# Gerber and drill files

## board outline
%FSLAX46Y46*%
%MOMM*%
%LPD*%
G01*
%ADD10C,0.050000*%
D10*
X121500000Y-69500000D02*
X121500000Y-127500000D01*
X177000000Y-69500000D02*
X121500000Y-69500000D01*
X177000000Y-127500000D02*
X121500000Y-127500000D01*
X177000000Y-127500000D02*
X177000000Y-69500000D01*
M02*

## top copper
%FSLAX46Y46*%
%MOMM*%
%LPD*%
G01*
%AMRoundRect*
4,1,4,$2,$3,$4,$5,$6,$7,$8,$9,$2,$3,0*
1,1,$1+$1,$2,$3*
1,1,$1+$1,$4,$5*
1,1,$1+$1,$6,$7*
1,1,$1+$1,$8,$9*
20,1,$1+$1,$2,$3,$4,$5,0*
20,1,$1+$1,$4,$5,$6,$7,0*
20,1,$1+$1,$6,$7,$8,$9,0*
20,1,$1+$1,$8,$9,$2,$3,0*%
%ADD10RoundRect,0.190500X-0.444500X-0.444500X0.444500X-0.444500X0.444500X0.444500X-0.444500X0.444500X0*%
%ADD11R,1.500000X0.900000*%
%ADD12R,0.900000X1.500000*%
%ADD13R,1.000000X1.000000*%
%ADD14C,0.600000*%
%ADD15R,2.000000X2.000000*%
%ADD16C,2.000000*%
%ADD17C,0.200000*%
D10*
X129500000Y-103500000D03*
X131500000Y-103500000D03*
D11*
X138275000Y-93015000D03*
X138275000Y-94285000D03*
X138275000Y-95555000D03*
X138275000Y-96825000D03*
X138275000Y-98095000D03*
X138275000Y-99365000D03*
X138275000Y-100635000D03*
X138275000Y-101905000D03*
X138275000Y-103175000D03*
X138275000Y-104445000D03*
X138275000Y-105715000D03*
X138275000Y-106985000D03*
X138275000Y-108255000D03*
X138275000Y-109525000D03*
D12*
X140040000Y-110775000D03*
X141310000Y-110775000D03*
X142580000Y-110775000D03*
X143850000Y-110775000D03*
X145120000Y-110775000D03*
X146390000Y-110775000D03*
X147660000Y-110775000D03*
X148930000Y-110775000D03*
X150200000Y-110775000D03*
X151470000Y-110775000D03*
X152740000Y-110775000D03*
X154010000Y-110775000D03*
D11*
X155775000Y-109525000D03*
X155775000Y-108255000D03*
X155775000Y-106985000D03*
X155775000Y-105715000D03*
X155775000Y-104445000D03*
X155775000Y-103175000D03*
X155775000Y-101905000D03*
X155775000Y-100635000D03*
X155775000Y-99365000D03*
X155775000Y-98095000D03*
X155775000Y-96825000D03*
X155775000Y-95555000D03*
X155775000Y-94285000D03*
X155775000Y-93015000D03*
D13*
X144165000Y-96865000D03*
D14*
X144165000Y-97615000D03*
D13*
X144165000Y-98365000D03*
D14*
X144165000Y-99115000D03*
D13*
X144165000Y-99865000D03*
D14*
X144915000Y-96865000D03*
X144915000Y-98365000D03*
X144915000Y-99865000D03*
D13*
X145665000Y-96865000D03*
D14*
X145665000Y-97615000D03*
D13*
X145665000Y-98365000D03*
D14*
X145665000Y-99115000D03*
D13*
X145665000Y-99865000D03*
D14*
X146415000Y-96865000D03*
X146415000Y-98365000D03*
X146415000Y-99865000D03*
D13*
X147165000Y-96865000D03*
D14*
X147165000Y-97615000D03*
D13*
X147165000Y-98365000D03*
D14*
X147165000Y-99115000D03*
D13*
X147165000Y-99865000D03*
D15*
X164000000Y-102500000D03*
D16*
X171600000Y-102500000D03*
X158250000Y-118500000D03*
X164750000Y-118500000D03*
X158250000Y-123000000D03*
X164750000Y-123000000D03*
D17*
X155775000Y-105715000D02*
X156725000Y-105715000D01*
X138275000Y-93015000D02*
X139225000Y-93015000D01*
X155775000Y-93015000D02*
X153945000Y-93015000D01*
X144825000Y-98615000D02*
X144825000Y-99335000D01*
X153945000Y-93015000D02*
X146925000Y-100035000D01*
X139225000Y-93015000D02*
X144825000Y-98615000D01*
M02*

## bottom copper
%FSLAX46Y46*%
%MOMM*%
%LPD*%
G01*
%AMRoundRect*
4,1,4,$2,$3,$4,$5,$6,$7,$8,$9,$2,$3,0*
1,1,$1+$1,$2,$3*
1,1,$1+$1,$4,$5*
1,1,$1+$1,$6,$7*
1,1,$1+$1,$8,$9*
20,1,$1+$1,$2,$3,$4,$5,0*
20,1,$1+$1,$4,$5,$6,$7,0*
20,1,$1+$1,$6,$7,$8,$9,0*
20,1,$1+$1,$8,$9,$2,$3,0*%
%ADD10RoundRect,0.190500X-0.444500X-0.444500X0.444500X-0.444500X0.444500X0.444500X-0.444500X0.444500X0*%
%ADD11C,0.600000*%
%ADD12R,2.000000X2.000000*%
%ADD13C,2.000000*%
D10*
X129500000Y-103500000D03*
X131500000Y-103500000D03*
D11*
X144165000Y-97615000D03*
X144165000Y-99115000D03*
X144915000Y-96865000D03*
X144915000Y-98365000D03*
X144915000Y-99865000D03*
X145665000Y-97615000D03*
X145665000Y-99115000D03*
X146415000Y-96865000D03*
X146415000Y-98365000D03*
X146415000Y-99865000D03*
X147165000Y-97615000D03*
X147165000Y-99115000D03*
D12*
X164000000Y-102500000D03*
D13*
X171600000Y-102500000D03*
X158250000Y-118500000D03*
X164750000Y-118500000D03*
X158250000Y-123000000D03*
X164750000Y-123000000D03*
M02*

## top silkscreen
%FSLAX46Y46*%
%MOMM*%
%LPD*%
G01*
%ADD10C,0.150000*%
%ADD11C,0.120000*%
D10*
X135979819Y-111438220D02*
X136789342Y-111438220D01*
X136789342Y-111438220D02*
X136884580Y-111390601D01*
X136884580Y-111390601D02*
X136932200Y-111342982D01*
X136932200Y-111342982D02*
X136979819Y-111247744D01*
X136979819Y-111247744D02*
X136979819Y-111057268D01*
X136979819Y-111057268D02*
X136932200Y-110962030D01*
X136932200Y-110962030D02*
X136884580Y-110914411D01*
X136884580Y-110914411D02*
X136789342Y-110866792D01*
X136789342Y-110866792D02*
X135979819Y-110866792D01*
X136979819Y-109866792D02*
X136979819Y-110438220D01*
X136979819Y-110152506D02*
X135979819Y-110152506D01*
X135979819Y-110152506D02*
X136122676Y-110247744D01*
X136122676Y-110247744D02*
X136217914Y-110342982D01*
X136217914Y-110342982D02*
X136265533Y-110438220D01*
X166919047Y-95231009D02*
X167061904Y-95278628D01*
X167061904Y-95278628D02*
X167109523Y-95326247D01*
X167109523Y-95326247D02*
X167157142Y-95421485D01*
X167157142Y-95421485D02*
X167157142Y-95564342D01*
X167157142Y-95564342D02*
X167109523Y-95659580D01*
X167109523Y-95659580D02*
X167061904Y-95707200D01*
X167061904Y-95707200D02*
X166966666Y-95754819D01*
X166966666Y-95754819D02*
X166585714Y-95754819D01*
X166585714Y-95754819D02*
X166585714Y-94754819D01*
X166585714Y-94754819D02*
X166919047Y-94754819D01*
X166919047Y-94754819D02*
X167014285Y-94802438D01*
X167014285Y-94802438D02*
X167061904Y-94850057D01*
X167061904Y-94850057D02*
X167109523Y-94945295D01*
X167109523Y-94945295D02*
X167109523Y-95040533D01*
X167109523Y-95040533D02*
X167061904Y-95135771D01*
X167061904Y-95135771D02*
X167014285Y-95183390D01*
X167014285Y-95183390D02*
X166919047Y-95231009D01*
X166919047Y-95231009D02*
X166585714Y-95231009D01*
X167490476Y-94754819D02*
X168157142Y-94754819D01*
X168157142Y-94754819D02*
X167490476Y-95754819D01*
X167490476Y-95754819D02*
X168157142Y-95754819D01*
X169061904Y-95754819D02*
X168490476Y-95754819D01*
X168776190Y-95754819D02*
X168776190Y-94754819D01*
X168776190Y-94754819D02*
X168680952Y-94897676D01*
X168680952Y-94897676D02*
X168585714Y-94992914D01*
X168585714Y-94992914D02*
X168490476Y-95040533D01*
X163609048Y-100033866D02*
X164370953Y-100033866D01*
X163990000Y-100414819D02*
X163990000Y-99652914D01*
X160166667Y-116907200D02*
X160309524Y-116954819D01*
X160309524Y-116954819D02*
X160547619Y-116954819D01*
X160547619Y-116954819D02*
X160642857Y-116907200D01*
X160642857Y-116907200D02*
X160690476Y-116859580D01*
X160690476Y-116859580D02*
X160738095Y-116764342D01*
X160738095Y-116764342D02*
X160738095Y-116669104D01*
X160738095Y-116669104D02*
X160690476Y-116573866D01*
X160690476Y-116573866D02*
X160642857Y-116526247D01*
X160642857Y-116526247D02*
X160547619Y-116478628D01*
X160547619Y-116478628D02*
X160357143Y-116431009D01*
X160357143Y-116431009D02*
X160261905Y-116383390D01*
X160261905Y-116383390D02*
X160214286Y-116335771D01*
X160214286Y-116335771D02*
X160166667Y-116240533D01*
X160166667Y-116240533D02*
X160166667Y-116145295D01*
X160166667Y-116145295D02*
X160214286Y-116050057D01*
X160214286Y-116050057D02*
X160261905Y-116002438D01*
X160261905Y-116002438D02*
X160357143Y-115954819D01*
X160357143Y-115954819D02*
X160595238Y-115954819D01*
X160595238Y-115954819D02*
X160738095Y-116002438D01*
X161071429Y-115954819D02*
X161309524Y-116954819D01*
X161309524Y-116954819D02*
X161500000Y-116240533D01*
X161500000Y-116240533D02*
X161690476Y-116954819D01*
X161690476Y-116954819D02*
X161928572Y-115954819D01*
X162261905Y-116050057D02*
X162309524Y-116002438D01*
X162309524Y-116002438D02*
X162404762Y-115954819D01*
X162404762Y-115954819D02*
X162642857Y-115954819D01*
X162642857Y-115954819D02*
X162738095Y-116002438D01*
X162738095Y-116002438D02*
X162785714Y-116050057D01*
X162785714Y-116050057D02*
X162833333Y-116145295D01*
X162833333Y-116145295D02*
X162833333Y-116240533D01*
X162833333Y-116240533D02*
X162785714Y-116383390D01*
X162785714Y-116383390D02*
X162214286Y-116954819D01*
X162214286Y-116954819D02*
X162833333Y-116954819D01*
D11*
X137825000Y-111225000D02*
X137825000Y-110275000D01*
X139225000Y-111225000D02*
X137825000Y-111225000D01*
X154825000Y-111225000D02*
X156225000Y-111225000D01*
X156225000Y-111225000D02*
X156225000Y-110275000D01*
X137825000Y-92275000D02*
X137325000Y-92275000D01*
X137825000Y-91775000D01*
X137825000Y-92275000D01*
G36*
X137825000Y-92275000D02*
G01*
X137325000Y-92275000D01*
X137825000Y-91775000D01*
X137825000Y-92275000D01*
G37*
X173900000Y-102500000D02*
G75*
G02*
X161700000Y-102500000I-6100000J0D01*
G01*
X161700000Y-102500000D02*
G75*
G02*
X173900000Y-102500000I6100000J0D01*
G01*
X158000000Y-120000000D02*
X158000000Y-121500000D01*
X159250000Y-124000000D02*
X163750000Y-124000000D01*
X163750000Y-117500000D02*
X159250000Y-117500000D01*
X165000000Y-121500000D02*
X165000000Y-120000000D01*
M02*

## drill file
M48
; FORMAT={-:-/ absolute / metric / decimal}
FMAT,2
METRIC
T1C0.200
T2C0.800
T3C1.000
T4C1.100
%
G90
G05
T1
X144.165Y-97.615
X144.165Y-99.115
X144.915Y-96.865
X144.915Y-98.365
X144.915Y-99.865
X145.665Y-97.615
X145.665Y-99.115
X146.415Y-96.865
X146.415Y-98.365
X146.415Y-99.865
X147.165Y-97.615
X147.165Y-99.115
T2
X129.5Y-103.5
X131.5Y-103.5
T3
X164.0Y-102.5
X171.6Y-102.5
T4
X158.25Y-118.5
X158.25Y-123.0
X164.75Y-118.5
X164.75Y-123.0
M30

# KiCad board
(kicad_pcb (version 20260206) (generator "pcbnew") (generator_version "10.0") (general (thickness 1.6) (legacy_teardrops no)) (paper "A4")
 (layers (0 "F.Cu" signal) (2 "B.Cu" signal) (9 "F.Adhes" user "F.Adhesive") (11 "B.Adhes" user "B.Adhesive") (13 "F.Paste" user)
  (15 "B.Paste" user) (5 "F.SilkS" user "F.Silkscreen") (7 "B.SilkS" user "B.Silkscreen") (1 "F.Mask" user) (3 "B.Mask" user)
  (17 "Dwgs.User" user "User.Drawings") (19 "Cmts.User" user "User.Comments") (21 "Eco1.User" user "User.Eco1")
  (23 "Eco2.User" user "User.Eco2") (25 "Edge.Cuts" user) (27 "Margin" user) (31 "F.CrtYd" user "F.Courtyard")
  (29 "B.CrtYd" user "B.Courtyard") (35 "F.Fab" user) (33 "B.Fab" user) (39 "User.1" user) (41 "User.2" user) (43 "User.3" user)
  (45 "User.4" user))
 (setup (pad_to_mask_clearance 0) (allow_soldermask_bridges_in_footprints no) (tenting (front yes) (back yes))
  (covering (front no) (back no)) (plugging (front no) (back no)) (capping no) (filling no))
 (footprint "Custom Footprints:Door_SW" (layer "F.Cu") (at 130.5 107.5)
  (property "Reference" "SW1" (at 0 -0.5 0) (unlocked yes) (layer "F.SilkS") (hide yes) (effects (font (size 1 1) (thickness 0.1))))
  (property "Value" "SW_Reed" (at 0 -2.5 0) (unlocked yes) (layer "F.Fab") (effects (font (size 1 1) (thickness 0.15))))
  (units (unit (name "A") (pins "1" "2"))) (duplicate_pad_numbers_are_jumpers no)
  (pad "1" thru_hole roundrect (at -1 -4) (size 1.27 1.27) (drill 0.8) (layers "*.Cu" "*.Mask") (remove_unused_layers no)
   (roundrect_rratio 0.15) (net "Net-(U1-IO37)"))
  (pad "2" thru_hole roundrect (at 1 -4) (size 1.27 1.27) (drill 0.8) (layers "*.Cu" "*.Mask") (remove_unused_layers no)
   (roundrect_rratio 0.15) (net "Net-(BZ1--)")))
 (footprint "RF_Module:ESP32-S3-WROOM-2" (layer "F.Cu") (at 147.025 98.275)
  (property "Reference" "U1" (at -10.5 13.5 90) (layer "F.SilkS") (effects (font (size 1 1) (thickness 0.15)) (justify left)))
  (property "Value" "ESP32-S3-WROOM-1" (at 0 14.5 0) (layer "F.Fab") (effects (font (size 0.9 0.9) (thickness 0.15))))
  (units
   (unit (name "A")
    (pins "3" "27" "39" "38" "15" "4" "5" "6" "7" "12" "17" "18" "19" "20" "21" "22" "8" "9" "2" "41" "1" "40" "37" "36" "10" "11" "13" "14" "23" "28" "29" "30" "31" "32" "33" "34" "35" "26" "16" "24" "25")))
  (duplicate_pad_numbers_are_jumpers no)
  (fp_line (start -9.2 12.95) (end -9.2 12) (stroke (width 0.12) (type solid)) (layer "F.SilkS"))
  (fp_line (start -7.8 12.95) (end -9.2 12.95) (stroke (width 0.12) (type solid)) (layer "F.SilkS"))
  (fp_line (start 7.8 12.95) (end 9.2 12.95) (stroke (width 0.12) (type solid)) (layer "F.SilkS"))
  (fp_line (start 9.2 12.95) (end 9.2 12) (stroke (width 0.12) (type solid)) (layer "F.SilkS"))
  (fp_poly (pts (xy -9.2 -6) (xy -9.7 -6) (xy -9.2 -6.5) (xy -9.2 -6)) (stroke (width 0.12) (type solid)) (fill yes) (layer "F.SilkS"))
  (pad "1" smd rect (at -8.75 -5.26) (size 1.5 0.9) (layers "F.Cu" "F.Mask" "F.Paste") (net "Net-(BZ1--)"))
  (pad "2" smd rect (at -8.75 -3.99) (size 1.5 0.9) (layers "F.Cu" "F.Mask" "F.Paste") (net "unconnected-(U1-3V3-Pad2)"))
  (pad "3" smd rect (at -8.75 -2.72) (size 1.5 0.9) (layers "F.Cu" "F.Mask" "F.Paste") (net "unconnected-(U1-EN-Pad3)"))
  (pad "4" smd rect (at -8.75 -1.45) (size 1.5 0.9) (layers "F.Cu" "F.Mask" "F.Paste") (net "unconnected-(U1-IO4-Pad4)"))
  (pad "5" smd rect (at -8.75 -0.18) (size 1.5 0.9) (layers "F.Cu" "F.Mask" "F.Paste") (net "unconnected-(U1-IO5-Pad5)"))
  (pad "6" smd rect (at -8.75 1.09) (size 1.5 0.9) (layers "F.Cu" "F.Mask" "F.Paste") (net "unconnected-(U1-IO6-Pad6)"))
  (pad "7" smd rect (at -8.75 2.36) (size 1.5 0.9) (layers "F.Cu" "F.Mask" "F.Paste") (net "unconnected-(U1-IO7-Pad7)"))
  (pad "8" smd rect (at -8.75 3.63) (size 1.5 0.9) (layers "F.Cu" "F.Mask" "F.Paste") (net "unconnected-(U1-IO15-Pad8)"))
  (pad "9" smd rect (at -8.75 4.9) (size 1.5 0.9) (layers "F.Cu" "F.Mask" "F.Paste") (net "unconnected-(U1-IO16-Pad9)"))
  (pad "10" smd rect (at -8.75 6.17) (size 1.5 0.9) (layers "F.Cu" "F.Mask" "F.Paste") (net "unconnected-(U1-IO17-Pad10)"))
  (pad "11" smd rect (at -8.75 7.44) (size 1.5 0.9) (layers "F.Cu" "F.Mask" "F.Paste") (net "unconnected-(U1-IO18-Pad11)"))
  (pad "12" smd rect (at -8.75 8.71) (size 1.5 0.9) (layers "F.Cu" "F.Mask" "F.Paste") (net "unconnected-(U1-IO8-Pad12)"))
  (pad "13" smd rect (at -8.75 9.98) (size 1.5 0.9) (layers "F.Cu" "F.Mask" "F.Paste") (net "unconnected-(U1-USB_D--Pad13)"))
  (pad "14" smd rect (at -8.75 11.25) (size 1.5 0.9) (layers "F.Cu" "F.Mask" "F.Paste") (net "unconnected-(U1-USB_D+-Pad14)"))
  (pad "15" smd rect (at -6.985 12.5 90) (size 1.5 0.9) (layers "F.Cu" "F.Mask" "F.Paste") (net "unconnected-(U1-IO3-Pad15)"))
  (pad "16" smd rect (at -5.715 12.5 90) (size 1.5 0.9) (layers "F.Cu" "F.Mask" "F.Paste") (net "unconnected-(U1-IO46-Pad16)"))
  (pad "17" smd rect (at -4.445 12.5 90) (size 1.5 0.9) (layers "F.Cu" "F.Mask" "F.Paste") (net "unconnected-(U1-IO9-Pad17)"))
  (pad "18" smd rect (at -3.175 12.5 90) (size 1.5 0.9) (layers "F.Cu" "F.Mask" "F.Paste") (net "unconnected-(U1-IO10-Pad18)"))
  (pad "19" smd rect (at -1.905 12.5 90) (size 1.5 0.9) (layers "F.Cu" "F.Mask" "F.Paste") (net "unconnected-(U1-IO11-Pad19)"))
  (pad "20" smd rect (at -0.635 12.5 90) (size 1.5 0.9) (layers "F.Cu" "F.Mask" "F.Paste") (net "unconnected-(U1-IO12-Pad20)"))
  (pad "21" smd rect (at 0.635 12.5 90) (size 1.5 0.9) (layers "F.Cu" "F.Mask" "F.Paste") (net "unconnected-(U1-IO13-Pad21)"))
  (pad "22" smd rect (at 1.905 12.5 90) (size 1.5 0.9) (layers "F.Cu" "F.Mask" "F.Paste") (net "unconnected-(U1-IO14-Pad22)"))
  (pad "23" smd rect (at 3.175 12.5 90) (size 1.5 0.9) (layers "F.Cu" "F.Mask" "F.Paste") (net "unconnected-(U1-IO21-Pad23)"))
  (pad "24" smd rect (at 4.445 12.5 90) (size 1.5 0.9) (layers "F.Cu" "F.Mask" "F.Paste") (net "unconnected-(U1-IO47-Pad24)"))
  (pad "25" smd rect (at 5.715 12.5 90) (size 1.5 0.9) (layers "F.Cu" "F.Mask" "F.Paste") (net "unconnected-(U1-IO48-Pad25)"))
  (pad "26" smd rect (at 6.985 12.5 90) (size 1.5 0.9) (layers "F.Cu" "F.Mask" "F.Paste") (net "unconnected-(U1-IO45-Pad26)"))
  (pad "27" smd rect (at 8.75 11.25) (size 1.5 0.9) (layers "F.Cu" "F.Mask" "F.Paste") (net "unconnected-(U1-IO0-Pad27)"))
  (pad "28" smd rect (at 8.75 9.98) (size 1.5 0.9) (layers "F.Cu" "F.Mask" "F.Paste") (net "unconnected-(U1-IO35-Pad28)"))
  (pad "29" smd rect (at 8.75 8.71) (size 1.5 0.9) (layers "F.Cu" "F.Mask" "F.Paste") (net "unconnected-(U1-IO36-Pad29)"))
  (pad "30" smd rect (at 8.75 7.44) (size 1.5 0.9) (layers "F.Cu" "F.Mask" "F.Paste") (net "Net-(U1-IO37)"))
  (pad "31" smd rect (at 8.75 6.17) (size 1.5 0.9) (layers "F.Cu" "F.Mask" "F.Paste") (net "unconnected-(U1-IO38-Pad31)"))
  (pad "32" smd rect (at 8.75 4.9) (size 1.5 0.9) (layers "F.Cu" "F.Mask" "F.Paste") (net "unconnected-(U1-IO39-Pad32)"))
  (pad "33" smd rect (at 8.75 3.63) (size 1.5 0.9) (layers "F.Cu" "F.Mask" "F.Paste") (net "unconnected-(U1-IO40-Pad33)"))
  (pad "34" smd rect (at 8.75 2.36) (size 1.5 0.9) (layers "F.Cu" "F.Mask" "F.Paste") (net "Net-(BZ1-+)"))
  (pad "35" smd rect (at 8.75 1.09) (size 1.5 0.9) (layers "F.Cu" "F.Mask" "F.Paste") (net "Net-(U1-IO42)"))
  (pad "36" smd rect (at 8.75 -0.18) (size 1.5 0.9) (layers "F.Cu" "F.Mask" "F.Paste") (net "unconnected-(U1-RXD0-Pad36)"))
  (pad "37" smd rect (at 8.75 -1.45) (size 1.5 0.9) (layers "F.Cu" "F.Mask" "F.Paste") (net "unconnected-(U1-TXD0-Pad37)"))
  (pad "38" smd rect (at 8.75 -2.72) (size 1.5 0.9) (layers "F.Cu" "F.Mask" "F.Paste") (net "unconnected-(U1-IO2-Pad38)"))
  (pad "39" smd rect (at 8.75 -3.99) (size 1.5 0.9) (layers "F.Cu" "F.Mask" "F.Paste") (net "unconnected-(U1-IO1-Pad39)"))
  (pad "40" smd rect (at 8.75 -5.26) (size 1.5 0.9) (layers "F.Cu" "F.Mask" "F.Paste") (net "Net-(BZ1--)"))
  (pad "41" smd rect (at -2.86 -1.41) (size 1 1) (layers "F.Cu" "F.Mask" "F.Paste") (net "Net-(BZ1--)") (zone_connect 2)
   (thermal_bridge_angle 45))
  (pad "41" thru_hole circle (at -2.86 -0.66) (size 0.6 0.6) (drill 0.2) (layers "*.Cu" "*.Mask") (remove_unused_layers no)
   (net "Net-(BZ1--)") (zone_connect 2))
  (pad "41" smd rect (at -2.86 0.09) (size 1 1) (layers "F.Cu" "F.Mask" "F.Paste") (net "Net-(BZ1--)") (zone_connect 2)
   (thermal_bridge_angle 45))
  (pad "41" thru_hole circle (at -2.86 0.84) (size 0.6 0.6) (drill 0.2) (layers "*.Cu" "*.Mask") (remove_unused_layers no)
   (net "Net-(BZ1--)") (zone_connect 2))
  (pad "41" smd rect (at -2.86 1.59) (size 1 1) (layers "F.Cu" "F.Mask" "F.Paste") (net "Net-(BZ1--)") (zone_connect 2)
   (thermal_bridge_angle 45))
  (pad "41" thru_hole circle (at -2.11 -1.41) (size 0.6 0.6) (drill 0.2) (layers "*.Cu" "*.Mask") (remove_unused_layers no)
   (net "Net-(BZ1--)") (zone_connect 2))
  (pad "41" thru_hole circle (at -2.11 0.09) (size 0.6 0.6) (drill 0.2) (layers "*.Cu" "*.Mask") (remove_unused_layers no)
   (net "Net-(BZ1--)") (zone_connect 2))
  (pad "41" thru_hole circle (at -2.11 1.59) (size 0.6 0.6) (drill 0.2) (layers "*.Cu" "*.Mask") (remove_unused_layers no)
   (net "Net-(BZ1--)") (zone_connect 2))
  (pad "41" smd rect (at -1.36 -1.41) (size 1 1) (layers "F.Cu" "F.Mask" "F.Paste") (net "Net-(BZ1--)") (zone_connect 2)
   (thermal_bridge_angle 45))
  (pad "41" thru_hole circle (at -1.36 -0.66) (size 0.6 0.6) (drill 0.2) (layers "*.Cu" "*.Mask") (remove_unused_layers no)
   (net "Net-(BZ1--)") (zone_connect 2))
  (pad "41" smd rect (at -1.36 0.09) (size 1 1) (layers "F.Cu" "F.Mask" "F.Paste") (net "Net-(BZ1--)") (zone_connect 2)
   (thermal_bridge_angle 45))
  (pad "41" thru_hole circle (at -1.36 0.84) (size 0.6 0.6) (drill 0.2) (layers "*.Cu" "*.Mask") (remove_unused_layers no)
   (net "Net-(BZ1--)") (zone_connect 2))
  (pad "41" smd rect (at -1.36 1.59) (size 1 1) (layers "F.Cu" "F.Mask" "F.Paste") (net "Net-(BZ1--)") (zone_connect 2)
   (thermal_bridge_angle 45))
  (pad "41" thru_hole circle (at -0.61 -1.41) (size 0.6 0.6) (drill 0.2) (layers "*.Cu" "*.Mask") (remove_unused_layers no)
   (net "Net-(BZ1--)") (zone_connect 2))
  (pad "41" thru_hole circle (at -0.61 0.09) (size 0.6 0.6) (drill 0.2) (layers "*.Cu" "*.Mask") (remove_unused_layers no)
   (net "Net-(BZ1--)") (zone_connect 2))
  (pad "41" thru_hole circle (at -0.61 1.59) (size 0.6 0.6) (drill 0.2) (layers "*.Cu" "*.Mask") (remove_unused_layers no)
   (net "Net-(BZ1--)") (zone_connect 2))
  (pad "41" smd rect (at 0.14 -1.41) (size 1 1) (layers "F.Cu" "F.Mask" "F.Paste") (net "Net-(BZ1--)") (zone_connect 2)
   (thermal_bridge_angle 45))
  (pad "41" thru_hole circle (at 0.14 -0.66) (size 0.6 0.6) (drill 0.2) (layers "*.Cu" "*.Mask") (remove_unused_layers no)
   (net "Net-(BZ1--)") (zone_connect 2))
  (pad "41" smd rect (at 0.14 0.09) (size 1 1) (layers "F.Cu" "F.Mask" "F.Paste") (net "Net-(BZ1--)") (zone_connect 2)
   (thermal_bridge_angle 45))
  (pad "41" thru_hole circle (at 0.14 0.84) (size 0.6 0.6) (drill 0.2) (layers "*.Cu" "*.Mask") (remove_unused_layers no)
   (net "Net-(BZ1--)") (zone_connect 2))
  (pad "41" smd rect (at 0.14 1.59) (size 1 1) (layers "F.Cu" "F.Mask" "F.Paste") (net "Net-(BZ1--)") (zone_connect 2)
   (thermal_bridge_angle 45))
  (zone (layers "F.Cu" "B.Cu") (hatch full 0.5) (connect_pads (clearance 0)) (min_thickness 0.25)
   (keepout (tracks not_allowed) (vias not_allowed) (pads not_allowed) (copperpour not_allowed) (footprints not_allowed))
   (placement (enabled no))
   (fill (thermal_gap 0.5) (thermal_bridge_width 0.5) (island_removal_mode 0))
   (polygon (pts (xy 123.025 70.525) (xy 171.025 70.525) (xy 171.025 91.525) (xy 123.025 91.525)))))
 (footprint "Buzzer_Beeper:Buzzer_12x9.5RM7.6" (layer "F.Cu") (at 164 102.5)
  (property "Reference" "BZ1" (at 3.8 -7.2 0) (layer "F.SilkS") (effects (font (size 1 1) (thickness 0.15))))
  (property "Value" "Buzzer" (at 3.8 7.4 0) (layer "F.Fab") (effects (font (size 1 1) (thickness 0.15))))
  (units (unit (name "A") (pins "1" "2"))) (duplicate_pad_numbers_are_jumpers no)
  (fp_circle (center 3.8 0) (end 9.9 0) (stroke (width 0.12) (type solid)) (fill no) (layer "F.SilkS"))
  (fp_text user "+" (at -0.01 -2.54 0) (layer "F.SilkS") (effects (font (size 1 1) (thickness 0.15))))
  (pad "1" thru_hole rect (at 0 0) (size 2 2) (drill 1) (layers "*.Cu" "*.Mask") (remove_unused_layers no) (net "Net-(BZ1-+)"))
  (pad "2" thru_hole circle (at 7.6 0) (size 2 2) (drill 1) (layers "*.Cu" "*.Mask") (remove_unused_layers no) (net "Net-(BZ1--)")))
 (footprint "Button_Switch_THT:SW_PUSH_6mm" (layer "F.Cu") (at 158.25 118.5)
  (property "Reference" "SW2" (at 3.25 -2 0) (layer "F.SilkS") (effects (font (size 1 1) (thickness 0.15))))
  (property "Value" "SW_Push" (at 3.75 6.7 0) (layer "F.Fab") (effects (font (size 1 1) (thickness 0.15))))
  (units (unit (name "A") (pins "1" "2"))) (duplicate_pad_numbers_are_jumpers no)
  (fp_line (start -0.25 1.5) (end -0.25 3) (stroke (width 0.12) (type solid)) (layer "F.SilkS"))
  (fp_line (start 1 5.5) (end 5.5 5.5) (stroke (width 0.12) (type solid)) (layer "F.SilkS"))
  (fp_line (start 5.5 -1) (end 1 -1) (stroke (width 0.12) (type solid)) (layer "F.SilkS"))
  (fp_line (start 6.75 3) (end 6.75 1.5) (stroke (width 0.12) (type solid)) (layer "F.SilkS"))
  (pad "1" thru_hole circle (at 0 0 90) (size 2 2) (drill 1.1) (layers "*.Cu" "*.Mask") (remove_unused_layers no) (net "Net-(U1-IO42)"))
  (pad "1" thru_hole circle (at 6.5 0 90) (size 2 2) (drill 1.1) (layers "*.Cu" "*.Mask") (remove_unused_layers no) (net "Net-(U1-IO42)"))
  (pad "2" thru_hole circle (at 0 4.5 90) (size 2 2) (drill 1.1) (layers "*.Cu" "*.Mask") (remove_unused_layers no) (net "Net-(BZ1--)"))
  (pad "2" thru_hole circle (at 6.5 4.5 90) (size 2 2) (drill 1.1) (layers "*.Cu" "*.Mask") (remove_unused_layers no) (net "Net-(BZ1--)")))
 (gr_line (start 121.5 69.5) (end 121.5 127.5) (stroke (width 0.05) (type default)) (layer "Edge.Cuts"))
 (gr_line (start 177 69.5) (end 121.5 69.5) (stroke (width 0.05) (type default)) (layer "Edge.Cuts"))
 (gr_line (start 177 127.5) (end 121.5 127.5) (stroke (width 0.05) (type default)) (layer "Edge.Cuts"))
 (gr_line (start 177 127.5) (end 177 69.5) (stroke (width 0.05) (type default)) (layer "Edge.Cuts"))
 (segment (start 155.775 105.715) (end 156.725 105.715) (width 0.2) (layer "F.Cu") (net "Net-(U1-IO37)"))
 (segment (start 138.275 93.015) (end 139.225 93.015) (width 0.2) (layer "F.Cu") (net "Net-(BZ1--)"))
 (segment (start 155.775 93.015) (end 153.945 93.015) (width 0.2) (layer "F.Cu") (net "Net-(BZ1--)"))
 (segment (start 144.825 98.615) (end 144.825 99.335) (width 0.2) (layer "F.Cu") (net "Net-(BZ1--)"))
 (segment (start 153.945 93.015) (end 146.925 100.035) (width 0.2) (layer "F.Cu") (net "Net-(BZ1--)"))
 (segment (start 139.225 93.015) (end 144.825 98.615) (width 0.2) (layer "F.Cu") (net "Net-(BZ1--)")))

